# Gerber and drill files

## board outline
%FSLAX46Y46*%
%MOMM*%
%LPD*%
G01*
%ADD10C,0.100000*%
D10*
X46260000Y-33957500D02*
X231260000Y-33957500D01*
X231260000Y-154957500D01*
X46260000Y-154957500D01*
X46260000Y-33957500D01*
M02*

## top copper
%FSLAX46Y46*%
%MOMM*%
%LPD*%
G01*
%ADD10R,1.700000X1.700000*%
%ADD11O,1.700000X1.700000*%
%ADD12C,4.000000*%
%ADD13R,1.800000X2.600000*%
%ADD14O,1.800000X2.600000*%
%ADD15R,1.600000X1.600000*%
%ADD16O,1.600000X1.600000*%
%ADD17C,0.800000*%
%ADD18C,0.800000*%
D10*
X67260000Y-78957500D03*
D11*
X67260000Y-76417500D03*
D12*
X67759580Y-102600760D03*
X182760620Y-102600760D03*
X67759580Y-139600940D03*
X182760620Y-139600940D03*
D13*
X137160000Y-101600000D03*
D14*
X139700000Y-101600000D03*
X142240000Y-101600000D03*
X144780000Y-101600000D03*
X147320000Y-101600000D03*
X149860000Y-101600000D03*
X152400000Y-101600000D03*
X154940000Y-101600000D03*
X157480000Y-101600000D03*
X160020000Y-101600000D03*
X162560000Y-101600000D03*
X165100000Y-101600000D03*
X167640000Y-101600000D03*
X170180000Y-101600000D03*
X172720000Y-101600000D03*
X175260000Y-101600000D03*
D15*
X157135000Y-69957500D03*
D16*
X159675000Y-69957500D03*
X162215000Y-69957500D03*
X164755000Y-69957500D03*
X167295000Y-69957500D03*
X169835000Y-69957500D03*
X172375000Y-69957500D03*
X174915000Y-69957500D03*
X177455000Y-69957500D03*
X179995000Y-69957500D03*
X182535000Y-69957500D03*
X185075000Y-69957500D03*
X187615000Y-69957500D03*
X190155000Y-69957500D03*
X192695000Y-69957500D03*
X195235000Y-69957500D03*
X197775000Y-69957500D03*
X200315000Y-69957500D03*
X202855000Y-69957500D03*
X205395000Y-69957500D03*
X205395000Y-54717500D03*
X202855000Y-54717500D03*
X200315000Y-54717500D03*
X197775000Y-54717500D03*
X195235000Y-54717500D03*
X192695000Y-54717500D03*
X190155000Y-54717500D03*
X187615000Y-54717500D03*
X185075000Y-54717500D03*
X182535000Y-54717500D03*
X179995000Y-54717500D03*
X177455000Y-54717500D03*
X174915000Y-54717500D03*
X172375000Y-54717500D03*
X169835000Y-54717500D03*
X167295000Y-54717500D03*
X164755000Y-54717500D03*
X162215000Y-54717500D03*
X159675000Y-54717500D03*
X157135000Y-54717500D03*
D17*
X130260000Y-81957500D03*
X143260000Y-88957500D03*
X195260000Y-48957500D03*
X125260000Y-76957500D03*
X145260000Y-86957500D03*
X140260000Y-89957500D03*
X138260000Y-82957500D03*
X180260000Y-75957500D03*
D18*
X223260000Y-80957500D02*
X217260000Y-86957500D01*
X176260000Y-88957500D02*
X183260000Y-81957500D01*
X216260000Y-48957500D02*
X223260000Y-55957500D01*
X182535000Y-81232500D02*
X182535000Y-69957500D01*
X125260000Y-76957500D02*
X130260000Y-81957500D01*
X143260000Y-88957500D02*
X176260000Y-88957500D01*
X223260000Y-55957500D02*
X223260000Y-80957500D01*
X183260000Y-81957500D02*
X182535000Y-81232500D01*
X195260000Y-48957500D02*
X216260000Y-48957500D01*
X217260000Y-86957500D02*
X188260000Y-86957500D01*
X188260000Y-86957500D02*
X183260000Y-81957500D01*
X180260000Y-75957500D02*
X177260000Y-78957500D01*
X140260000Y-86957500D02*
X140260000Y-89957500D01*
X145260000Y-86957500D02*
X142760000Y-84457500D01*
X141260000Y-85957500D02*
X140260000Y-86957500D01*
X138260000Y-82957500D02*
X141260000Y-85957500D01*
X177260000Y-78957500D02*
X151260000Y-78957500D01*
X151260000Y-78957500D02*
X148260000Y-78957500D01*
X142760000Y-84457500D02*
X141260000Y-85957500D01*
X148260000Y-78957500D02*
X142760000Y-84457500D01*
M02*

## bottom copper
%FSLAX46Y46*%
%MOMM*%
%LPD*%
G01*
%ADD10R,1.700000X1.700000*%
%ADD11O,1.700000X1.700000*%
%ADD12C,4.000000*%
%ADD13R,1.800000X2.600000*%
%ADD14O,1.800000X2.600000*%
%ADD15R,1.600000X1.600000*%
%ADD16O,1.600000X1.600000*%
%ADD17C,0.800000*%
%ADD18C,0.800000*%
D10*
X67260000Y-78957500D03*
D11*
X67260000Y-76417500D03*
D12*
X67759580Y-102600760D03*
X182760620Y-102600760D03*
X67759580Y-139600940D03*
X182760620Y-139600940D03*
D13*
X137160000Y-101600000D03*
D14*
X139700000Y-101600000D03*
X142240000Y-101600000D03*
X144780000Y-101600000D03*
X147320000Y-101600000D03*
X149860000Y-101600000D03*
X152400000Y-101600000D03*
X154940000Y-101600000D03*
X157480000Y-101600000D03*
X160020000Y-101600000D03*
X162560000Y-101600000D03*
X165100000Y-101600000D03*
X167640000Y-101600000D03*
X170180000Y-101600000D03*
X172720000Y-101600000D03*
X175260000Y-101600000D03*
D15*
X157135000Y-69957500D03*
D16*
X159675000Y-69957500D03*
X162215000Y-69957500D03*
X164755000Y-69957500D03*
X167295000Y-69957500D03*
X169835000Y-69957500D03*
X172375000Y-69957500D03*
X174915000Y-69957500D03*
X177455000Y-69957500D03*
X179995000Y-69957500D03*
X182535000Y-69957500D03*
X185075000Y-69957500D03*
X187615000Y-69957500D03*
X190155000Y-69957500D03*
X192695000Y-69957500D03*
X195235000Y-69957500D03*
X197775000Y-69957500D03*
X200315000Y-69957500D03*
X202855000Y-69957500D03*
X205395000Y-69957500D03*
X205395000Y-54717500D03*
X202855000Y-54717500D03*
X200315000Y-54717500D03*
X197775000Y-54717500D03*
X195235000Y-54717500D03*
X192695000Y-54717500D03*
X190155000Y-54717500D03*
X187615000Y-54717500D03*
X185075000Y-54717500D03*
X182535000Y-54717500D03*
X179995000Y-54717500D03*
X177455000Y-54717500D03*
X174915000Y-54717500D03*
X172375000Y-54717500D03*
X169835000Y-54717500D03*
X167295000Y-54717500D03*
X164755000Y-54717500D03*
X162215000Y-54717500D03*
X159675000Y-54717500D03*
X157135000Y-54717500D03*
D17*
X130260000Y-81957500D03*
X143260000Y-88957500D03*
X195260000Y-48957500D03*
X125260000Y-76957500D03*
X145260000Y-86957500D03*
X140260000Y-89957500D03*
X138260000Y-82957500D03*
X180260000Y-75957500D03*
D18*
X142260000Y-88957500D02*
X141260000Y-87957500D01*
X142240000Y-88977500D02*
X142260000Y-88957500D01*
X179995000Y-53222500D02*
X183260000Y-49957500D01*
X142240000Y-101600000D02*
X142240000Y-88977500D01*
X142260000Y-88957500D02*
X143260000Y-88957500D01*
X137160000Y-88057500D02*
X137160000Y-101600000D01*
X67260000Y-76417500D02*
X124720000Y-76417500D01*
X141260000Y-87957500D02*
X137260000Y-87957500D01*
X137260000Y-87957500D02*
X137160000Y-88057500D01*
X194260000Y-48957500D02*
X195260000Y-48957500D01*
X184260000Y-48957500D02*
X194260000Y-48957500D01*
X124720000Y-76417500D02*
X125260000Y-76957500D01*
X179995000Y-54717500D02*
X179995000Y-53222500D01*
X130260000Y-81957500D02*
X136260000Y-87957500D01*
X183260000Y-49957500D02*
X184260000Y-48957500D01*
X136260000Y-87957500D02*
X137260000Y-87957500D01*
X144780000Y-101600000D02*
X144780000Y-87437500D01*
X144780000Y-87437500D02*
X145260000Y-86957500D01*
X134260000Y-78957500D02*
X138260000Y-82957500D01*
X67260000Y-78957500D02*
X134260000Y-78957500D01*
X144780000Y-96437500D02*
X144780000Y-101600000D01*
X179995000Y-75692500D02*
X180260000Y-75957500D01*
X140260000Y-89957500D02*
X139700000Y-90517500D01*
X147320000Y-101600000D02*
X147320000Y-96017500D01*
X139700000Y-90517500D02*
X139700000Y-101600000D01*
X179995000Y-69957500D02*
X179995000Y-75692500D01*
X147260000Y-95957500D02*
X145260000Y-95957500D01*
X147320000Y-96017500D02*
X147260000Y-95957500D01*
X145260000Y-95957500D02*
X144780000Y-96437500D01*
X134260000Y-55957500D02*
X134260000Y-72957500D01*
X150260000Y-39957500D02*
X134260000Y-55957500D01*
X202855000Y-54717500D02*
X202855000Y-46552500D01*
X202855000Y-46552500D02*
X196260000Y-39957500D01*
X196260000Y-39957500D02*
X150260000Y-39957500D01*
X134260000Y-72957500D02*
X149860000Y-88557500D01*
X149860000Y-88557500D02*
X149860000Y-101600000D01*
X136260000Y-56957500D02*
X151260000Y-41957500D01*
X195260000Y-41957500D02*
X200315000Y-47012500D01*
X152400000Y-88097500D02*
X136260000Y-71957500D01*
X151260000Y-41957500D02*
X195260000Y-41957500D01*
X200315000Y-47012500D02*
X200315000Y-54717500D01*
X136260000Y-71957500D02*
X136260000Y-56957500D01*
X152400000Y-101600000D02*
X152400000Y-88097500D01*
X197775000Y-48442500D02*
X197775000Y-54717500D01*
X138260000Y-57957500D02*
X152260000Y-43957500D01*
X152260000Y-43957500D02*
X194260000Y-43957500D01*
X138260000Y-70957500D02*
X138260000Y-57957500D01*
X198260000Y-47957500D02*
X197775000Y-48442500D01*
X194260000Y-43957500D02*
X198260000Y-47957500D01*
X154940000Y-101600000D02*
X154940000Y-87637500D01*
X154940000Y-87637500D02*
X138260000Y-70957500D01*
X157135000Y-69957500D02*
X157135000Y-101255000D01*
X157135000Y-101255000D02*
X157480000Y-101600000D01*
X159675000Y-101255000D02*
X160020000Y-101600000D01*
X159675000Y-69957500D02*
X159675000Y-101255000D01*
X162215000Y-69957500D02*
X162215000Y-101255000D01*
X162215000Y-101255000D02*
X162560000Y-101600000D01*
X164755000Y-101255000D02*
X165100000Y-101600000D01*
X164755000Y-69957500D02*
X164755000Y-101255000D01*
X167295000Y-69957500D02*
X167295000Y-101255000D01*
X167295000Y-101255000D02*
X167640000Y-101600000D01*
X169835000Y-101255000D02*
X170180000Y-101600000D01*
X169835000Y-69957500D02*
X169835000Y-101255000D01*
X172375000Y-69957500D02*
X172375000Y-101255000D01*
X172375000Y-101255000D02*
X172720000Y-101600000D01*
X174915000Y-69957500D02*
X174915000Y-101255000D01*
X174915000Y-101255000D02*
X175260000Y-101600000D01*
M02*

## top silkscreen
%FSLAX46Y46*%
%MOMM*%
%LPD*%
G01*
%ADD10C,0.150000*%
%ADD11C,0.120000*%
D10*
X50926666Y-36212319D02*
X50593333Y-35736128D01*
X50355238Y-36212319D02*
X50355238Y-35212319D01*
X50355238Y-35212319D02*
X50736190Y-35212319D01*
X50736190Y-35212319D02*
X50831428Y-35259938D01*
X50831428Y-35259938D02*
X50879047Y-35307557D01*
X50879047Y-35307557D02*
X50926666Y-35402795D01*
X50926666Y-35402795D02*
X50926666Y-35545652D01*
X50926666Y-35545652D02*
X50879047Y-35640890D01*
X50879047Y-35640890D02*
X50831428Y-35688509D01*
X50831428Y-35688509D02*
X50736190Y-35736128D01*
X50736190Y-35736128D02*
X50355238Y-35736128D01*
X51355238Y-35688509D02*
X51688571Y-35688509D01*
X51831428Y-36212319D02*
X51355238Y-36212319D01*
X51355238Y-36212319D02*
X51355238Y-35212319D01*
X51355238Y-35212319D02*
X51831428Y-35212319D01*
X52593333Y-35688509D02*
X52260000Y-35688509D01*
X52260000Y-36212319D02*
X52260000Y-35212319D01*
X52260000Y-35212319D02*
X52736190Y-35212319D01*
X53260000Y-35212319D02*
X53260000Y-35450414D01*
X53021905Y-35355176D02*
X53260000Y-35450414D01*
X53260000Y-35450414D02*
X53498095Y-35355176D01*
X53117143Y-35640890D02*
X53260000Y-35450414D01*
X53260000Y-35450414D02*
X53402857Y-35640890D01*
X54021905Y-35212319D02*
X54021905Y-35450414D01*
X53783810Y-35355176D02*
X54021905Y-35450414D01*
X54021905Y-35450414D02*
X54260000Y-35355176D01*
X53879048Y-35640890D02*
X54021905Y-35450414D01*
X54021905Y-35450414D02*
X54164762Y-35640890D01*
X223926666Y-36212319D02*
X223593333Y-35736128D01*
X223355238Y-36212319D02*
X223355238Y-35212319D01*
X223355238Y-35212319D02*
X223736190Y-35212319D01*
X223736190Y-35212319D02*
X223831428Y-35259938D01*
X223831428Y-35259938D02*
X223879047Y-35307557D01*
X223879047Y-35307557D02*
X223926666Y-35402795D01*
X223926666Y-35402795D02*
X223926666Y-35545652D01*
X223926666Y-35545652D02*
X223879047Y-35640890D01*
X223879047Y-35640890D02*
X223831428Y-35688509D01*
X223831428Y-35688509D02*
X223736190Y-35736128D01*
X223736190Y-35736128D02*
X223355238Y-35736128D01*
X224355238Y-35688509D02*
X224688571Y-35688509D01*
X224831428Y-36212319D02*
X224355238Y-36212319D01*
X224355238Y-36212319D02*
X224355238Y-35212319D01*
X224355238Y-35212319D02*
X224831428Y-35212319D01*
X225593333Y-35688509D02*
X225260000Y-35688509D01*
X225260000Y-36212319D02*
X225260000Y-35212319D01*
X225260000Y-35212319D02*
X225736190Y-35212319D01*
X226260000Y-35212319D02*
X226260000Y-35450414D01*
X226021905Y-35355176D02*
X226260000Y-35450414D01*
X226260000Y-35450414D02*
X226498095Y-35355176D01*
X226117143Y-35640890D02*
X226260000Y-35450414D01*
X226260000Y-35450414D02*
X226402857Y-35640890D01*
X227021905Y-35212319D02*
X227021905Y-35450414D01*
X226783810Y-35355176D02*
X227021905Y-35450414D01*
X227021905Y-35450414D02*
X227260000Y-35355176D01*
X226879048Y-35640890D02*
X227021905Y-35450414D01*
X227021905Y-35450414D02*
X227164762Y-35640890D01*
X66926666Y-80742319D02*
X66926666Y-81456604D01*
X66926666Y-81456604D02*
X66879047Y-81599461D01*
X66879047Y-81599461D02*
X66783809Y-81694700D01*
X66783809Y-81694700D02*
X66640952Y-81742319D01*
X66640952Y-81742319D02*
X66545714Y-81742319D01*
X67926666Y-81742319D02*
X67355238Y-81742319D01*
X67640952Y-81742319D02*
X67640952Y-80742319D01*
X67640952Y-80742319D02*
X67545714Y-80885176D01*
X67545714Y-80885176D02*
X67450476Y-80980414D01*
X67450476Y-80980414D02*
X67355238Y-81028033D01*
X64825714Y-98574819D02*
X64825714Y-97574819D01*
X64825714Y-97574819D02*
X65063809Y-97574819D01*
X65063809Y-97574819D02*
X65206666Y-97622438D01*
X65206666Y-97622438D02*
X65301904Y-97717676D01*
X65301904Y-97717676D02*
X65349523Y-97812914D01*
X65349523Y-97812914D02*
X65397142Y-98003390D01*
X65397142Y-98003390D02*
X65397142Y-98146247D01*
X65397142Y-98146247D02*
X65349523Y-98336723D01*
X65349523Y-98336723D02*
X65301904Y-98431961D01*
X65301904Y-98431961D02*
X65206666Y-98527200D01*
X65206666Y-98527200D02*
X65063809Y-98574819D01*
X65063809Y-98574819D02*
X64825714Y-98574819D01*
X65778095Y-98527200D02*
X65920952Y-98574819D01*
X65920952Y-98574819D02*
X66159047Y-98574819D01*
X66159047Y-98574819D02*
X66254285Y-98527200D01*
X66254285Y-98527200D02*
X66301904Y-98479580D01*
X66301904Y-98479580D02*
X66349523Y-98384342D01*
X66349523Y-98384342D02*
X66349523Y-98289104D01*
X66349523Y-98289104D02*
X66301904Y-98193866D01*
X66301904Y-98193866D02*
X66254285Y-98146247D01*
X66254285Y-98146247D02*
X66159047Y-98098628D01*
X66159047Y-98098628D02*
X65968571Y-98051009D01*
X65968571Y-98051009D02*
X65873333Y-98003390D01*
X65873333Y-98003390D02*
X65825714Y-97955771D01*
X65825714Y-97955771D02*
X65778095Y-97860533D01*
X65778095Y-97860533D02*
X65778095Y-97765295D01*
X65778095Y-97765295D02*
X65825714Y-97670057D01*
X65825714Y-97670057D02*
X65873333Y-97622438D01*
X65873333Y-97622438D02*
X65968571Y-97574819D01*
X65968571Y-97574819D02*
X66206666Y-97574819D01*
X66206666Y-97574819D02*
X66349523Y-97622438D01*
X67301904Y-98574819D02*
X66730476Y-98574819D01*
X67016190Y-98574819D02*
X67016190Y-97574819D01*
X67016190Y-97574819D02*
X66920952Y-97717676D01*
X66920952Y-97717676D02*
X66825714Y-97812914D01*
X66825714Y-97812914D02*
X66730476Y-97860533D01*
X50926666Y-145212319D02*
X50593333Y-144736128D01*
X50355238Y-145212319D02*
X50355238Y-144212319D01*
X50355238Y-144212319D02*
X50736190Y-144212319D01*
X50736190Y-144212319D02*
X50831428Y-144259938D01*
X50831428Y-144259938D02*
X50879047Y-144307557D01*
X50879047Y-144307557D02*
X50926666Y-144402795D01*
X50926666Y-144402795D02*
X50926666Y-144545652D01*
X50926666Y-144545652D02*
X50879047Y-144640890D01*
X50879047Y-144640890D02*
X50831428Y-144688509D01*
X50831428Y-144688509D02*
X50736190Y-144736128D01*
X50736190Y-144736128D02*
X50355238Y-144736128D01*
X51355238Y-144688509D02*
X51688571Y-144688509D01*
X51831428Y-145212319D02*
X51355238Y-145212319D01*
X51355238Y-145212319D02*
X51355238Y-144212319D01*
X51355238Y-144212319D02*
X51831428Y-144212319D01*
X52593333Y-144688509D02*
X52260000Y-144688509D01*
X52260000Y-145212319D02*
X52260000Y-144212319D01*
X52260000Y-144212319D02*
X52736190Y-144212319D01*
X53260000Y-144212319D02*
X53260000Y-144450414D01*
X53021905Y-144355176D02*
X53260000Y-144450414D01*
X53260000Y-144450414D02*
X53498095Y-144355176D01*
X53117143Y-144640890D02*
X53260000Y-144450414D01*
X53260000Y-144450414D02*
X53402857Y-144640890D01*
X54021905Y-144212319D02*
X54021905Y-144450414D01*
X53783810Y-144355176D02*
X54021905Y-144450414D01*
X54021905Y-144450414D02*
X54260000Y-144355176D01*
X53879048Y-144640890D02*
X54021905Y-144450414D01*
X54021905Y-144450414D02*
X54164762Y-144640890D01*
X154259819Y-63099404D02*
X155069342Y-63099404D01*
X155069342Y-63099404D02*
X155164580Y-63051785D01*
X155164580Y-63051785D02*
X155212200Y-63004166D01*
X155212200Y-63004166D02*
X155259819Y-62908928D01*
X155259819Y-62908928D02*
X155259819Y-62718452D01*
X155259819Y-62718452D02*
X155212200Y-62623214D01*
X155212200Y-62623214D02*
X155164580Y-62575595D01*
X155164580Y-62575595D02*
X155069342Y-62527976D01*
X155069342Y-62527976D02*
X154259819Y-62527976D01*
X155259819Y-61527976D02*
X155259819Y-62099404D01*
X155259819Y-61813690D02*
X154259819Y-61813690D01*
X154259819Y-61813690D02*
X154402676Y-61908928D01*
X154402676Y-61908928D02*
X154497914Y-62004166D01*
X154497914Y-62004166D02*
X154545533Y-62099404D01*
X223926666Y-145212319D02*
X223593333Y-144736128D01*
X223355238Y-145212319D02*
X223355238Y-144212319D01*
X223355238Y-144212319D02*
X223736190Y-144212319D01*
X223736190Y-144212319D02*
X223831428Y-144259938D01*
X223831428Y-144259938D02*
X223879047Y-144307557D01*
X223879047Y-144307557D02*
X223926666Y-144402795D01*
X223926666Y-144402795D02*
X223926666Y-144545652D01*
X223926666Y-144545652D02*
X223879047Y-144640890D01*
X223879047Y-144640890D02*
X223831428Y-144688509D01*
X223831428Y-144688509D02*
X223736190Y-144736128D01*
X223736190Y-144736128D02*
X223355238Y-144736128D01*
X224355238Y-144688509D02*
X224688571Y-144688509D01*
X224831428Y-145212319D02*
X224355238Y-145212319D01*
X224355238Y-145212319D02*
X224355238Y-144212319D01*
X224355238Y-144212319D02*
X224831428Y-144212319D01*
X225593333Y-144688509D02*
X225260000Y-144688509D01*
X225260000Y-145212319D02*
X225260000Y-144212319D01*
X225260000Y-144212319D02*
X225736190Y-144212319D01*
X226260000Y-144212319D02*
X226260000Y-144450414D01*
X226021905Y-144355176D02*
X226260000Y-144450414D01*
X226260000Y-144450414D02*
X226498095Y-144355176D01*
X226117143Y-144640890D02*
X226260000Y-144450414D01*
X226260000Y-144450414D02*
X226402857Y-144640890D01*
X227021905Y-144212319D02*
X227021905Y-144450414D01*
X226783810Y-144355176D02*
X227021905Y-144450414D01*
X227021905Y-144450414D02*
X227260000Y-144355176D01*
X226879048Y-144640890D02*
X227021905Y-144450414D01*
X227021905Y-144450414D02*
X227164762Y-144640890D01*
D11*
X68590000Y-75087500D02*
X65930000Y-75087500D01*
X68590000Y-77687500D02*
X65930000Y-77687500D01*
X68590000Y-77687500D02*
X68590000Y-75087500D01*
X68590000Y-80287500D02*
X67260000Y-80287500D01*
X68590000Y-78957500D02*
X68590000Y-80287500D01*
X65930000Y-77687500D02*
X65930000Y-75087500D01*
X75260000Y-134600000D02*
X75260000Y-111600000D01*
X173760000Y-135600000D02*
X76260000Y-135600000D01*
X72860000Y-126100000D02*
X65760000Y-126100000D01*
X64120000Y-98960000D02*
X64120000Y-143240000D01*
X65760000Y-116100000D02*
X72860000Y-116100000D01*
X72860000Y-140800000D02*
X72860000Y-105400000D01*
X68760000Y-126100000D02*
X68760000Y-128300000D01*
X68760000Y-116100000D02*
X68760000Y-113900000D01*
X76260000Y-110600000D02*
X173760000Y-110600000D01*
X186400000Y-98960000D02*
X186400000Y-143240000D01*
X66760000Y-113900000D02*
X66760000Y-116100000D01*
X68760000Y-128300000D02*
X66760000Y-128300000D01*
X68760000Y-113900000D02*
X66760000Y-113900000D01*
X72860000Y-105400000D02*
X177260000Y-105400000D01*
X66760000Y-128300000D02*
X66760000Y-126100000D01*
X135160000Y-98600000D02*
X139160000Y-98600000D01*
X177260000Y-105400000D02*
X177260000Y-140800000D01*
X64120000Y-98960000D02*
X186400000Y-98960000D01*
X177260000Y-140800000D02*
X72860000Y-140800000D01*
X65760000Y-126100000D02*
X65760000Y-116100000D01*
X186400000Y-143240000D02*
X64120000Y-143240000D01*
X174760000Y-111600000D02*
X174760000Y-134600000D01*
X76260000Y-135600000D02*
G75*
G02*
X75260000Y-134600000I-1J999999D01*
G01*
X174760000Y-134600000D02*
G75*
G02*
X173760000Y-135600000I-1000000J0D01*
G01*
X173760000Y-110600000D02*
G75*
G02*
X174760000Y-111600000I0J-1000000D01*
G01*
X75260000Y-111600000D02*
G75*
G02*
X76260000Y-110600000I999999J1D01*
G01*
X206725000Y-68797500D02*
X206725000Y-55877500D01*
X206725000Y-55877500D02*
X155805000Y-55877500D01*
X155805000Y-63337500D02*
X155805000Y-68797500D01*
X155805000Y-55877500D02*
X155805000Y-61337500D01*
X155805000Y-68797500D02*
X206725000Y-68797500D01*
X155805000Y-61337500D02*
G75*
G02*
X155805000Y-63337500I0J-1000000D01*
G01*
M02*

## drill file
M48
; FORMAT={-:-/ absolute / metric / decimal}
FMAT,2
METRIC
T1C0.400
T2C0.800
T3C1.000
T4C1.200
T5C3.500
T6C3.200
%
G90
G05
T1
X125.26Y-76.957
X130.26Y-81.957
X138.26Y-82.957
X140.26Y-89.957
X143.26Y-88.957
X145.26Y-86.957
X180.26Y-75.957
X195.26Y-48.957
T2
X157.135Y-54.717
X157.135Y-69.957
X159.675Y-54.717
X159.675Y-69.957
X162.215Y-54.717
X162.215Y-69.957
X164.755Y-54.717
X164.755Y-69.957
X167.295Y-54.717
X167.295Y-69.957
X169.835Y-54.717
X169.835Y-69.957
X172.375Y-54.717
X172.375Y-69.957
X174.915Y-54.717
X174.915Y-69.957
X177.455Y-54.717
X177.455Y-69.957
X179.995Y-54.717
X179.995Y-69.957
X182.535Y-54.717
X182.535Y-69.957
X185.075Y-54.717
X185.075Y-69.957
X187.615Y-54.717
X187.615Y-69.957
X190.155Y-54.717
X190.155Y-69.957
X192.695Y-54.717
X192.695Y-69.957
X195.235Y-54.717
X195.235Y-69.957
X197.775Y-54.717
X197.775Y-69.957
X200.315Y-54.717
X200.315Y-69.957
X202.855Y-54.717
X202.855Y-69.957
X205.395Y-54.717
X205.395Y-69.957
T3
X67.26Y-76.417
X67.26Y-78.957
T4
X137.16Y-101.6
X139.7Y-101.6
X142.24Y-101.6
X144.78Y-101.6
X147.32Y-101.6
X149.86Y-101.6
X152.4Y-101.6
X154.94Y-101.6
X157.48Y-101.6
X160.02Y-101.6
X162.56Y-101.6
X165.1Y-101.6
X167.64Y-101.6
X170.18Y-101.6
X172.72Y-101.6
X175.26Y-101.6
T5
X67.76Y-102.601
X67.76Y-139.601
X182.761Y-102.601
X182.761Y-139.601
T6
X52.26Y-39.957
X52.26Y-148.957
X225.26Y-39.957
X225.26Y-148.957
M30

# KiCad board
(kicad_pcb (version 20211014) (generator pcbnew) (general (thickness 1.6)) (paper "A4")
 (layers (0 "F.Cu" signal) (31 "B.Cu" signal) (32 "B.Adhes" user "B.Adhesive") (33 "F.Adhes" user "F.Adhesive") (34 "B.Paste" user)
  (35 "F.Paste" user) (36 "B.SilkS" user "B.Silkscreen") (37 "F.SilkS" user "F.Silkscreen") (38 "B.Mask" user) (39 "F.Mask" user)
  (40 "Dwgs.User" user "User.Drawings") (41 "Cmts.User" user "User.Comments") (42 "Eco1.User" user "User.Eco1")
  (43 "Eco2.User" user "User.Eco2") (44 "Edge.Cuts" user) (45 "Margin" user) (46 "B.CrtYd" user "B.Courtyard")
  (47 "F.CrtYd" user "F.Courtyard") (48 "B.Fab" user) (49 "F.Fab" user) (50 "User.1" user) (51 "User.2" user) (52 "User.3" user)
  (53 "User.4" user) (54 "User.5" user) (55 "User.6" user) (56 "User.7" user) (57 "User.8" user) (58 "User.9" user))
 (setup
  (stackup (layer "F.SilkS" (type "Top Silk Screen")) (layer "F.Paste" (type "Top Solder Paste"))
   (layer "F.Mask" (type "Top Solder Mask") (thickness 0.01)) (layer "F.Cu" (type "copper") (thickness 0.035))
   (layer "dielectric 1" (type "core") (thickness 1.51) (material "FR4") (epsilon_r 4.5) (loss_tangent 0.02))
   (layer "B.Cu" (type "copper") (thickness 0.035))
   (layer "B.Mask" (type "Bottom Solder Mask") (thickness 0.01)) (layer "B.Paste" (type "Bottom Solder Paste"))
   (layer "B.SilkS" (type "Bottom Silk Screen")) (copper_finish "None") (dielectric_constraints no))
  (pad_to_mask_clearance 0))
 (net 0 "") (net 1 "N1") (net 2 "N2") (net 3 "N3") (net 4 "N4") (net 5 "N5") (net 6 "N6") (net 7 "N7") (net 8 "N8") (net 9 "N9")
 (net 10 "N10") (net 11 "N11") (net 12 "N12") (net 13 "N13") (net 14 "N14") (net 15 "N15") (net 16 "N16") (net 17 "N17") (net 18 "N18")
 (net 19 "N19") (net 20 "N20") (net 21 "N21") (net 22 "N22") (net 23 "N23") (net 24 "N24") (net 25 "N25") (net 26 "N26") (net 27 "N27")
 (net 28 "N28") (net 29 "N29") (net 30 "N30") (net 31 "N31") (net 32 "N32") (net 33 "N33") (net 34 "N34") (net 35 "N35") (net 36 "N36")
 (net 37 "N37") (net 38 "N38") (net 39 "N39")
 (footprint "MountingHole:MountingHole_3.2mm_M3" (layer "F.Cu") (at 52.26 39.9575)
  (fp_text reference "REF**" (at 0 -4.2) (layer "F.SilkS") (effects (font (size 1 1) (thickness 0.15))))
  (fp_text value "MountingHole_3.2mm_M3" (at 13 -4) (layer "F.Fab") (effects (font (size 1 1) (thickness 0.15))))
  (pad "" np_thru_hole circle (at 0 0) (size 3.2 3.2) (drill 3.2) (layers *.Cu *.Mask)))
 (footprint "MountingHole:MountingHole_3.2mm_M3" (layer "F.Cu") (at 225.26 39.9575)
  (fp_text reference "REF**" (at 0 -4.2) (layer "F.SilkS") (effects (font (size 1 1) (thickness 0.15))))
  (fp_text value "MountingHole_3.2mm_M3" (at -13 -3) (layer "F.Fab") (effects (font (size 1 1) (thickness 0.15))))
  (pad "" np_thru_hole circle (at 0 0) (size 3.2 3.2) (drill 3.2) (layers *.Cu *.Mask)))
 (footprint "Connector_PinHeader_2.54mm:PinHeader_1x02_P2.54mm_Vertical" (layer "F.Cu") (at 67.26 78.9575 180)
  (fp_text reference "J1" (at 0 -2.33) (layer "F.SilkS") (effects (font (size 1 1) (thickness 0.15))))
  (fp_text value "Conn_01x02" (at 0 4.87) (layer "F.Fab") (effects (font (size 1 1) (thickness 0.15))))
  (fp_line (start -1.33 3.87) (end 1.33 3.87) (layer "F.SilkS") (width 0.12))
  (fp_line (start -1.33 1.27) (end 1.33 1.27) (layer "F.SilkS") (width 0.12))
  (fp_line (start -1.33 1.27) (end -1.33 3.87) (layer "F.SilkS") (width 0.12))
  (fp_line (start -1.33 -1.33) (end 0 -1.33) (layer "F.SilkS") (width 0.12))
  (fp_line (start -1.33 0) (end -1.33 -1.33) (layer "F.SilkS") (width 0.12))
  (fp_line (start 1.33 1.27) (end 1.33 3.87) (layer "F.SilkS") (width 0.12))
  (pad "1" thru_hole rect (at 0 0 180) (size 1.7 1.7) (drill 1) (layers *.Cu *.Mask) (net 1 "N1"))
  (pad "2" thru_hole oval (at 0 2.54 180) (size 1.7 1.7) (drill 1) (layers *.Cu *.Mask) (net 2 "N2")))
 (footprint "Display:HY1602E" (layer "F.Cu") (at 137.16 101.6)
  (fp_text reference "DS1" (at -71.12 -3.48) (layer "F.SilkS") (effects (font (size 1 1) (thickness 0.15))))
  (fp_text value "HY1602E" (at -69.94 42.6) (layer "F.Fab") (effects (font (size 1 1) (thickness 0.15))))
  (fp_line (start -61.9 33) (end -61.9 10) (layer "F.SilkS") (width 0.12))
  (fp_line (start 36.6 34) (end -60.9 34) (layer "F.SilkS") (width 0.12))
  (fp_line (start -64.3 24.5) (end -71.4 24.5) (layer "F.SilkS") (width 0.12))
  (fp_line (start -73.04 -2.64) (end -73.04 41.64) (layer "F.SilkS") (width 0.12))
  (fp_line (start -71.4 14.5) (end -64.3 14.5) (layer "F.SilkS") (width 0.12))
  (fp_line (start -64.3 39.2) (end -64.3 3.8) (layer "F.SilkS") (width 0.12))
  (fp_line (start -68.4 24.5) (end -68.4 26.7) (layer "F.SilkS") (width 0.12))
  (fp_line (start -68.4 14.5) (end -68.4 12.3) (layer "F.SilkS") (width 0.12))
  (fp_line (start -60.9 9) (end 36.6 9) (layer "F.SilkS") (width 0.12))
  (fp_line (start 49.24 -2.64) (end 49.24 41.64) (layer "F.SilkS") (width 0.12))
  (fp_line (start -70.4 12.3) (end -70.4 14.5) (layer "F.SilkS") (width 0.12))
  (fp_line (start -68.4 26.7) (end -70.4 26.7) (layer "F.SilkS") (width 0.12))
  (fp_line (start -68.4 12.3) (end -70.4 12.3) (layer "F.SilkS") (width 0.12))
  (fp_line (start -64.3 3.8) (end 40.1 3.8) (layer "F.SilkS") (width 0.12))
  (fp_line (start -70.4 26.7) (end -70.4 24.5) (layer "F.SilkS") (width 0.12))
  (fp_line (start -2 -3) (end 2 -3) (layer "F.SilkS") (width 0.12))
  (fp_line (start 40.1 3.8) (end 40.1 39.2) (layer "F.SilkS") (width 0.12))
  (fp_line (start -73.04 -2.64) (end 49.24 -2.64) (layer "F.SilkS") (width 0.12))
  (fp_line (start 40.1 39.2) (end -64.3 39.2) (layer "F.SilkS") (width 0.12))
  (fp_line (start -71.4 24.5) (end -71.4 14.5) (layer "F.SilkS") (width 0.12))
  (fp_line (start 49.24 41.64) (end -73.04 41.64) (layer "F.SilkS") (width 0.12))
  (fp_line (start 37.6 10) (end 37.6 33) (layer "F.SilkS") (width 0.12))
  (fp_arc (start -60.9 34) (mid -61.607107 33.707107) (end -61.9 33) (layer "F.SilkS") (width 0.12))
  (fp_arc (start 37.6 33) (mid 37.307107 33.707107) (end 36.6 34) (layer "F.SilkS") (width 0.12))
  (fp_arc (start 36.6 9) (mid 37.307107 9.292893) (end 37.6 10) (layer "F.SilkS") (width 0.12))
  (fp_arc (start -61.9 10) (mid -61.607107 9.292893) (end -60.9 9) (layer "F.SilkS") (width 0.12))
  (pad "" thru_hole circle (at -69.40042 1.00076 180) (size 4 4) (drill 3.5) (layers *.Cu *.Mask))
  (pad "" thru_hole circle (at 45.60062 1.00076 180) (size 4 4) (drill 3.5) (layers *.Cu *.Mask))
  (pad "" thru_hole circle (at -69.40042 38.00094 180) (size 4 4) (drill 3.5) (layers *.Cu *.Mask))
  (pad "" thru_hole circle (at 45.60062 38.00094 180) (size 4 4) (drill 3.5) (layers *.Cu *.Mask))
  (pad "1" thru_hole rect (at 0 0 180) (size 1.8 2.6) (drill 1.2) (layers *.Cu *.Mask) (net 2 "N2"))
  (pad "2" thru_hole oval (at 2.54 0 180) (size 1.8 2.6) (drill 1.2) (layers *.Cu *.Mask) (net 1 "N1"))
  (pad "3" thru_hole oval (at 5.08 0 180) (size 1.8 2.6) (drill 1.2) (layers *.Cu *.Mask) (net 2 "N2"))
  (pad "4" thru_hole oval (at 7.62 0 180) (size 1.8 2.6) (drill 1.2) (layers *.Cu *.Mask) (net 1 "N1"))
  (pad "5" thru_hole oval (at 10.16 0 180) (size 1.8 2.6) (drill 1.2) (layers *.Cu *.Mask) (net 1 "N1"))
  (pad "6" thru_hole oval (at 12.7 0 180) (size 1.8 2.6) (drill 1.2) (layers *.Cu *.Mask) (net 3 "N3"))
  (pad "7" thru_hole oval (at 15.24 0 180) (size 1.8 2.6) (drill 1.2) (layers *.Cu *.Mask) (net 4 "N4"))
  (pad "8" thru_hole oval (at 17.78 0 180) (size 1.8 2.6) (drill 1.2) (layers *.Cu *.Mask) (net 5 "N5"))
  (pad "9" thru_hole oval (at 20.32 0 180) (size 1.8 2.6) (drill 1.2) (layers *.Cu *.Mask) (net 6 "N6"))
  (pad "10" thru_hole oval (at 22.86 0 180) (size 1.8 2.6) (drill 1.2) (layers *.Cu *.Mask) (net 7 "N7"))
  (pad "11" thru_hole oval (at 25.4 0 180) (size 1.8 2.6) (drill 1.2) (layers *.Cu *.Mask) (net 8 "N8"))
  (pad "12" thru_hole oval (at 27.94 0 180) (size 1.8 2.6) (drill 1.2) (layers *.Cu *.Mask) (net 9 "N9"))
  (pad "13" thru_hole oval (at 30.48 0 180) (size 1.8 2.6) (drill 1.2) (layers *.Cu *.Mask) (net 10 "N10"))
  (pad "14" thru_hole oval (at 33.02 0 180) (size 1.8 2.6) (drill 1.2) (layers *.Cu *.Mask) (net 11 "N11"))
  (pad "15" thru_hole oval (at 35.56 0 180) (size 1.8 2.6) (drill 1.2) (layers *.Cu *.Mask) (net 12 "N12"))
  (pad "16" thru_hole oval (at 38.1 0 180) (size 1.8 2.6) (drill 1.2) (layers *.Cu *.Mask) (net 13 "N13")))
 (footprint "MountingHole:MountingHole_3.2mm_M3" (layer "F.Cu") (at 52.26 148.9575)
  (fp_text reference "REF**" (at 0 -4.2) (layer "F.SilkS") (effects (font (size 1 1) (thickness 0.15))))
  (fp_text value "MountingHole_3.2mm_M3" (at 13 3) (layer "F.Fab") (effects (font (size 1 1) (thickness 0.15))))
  (pad "" np_thru_hole circle (at 0 0) (size 3.2 3.2) (drill 3.2) (layers *.Cu *.Mask)))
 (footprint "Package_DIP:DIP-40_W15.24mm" (layer "F.Cu") (at 157.135 69.9575 90)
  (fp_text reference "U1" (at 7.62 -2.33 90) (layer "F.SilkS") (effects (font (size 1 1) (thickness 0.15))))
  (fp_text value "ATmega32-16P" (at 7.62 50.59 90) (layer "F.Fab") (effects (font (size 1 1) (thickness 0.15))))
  (fp_line (start 1.16 49.59) (end 14.08 49.59) (layer "F.SilkS") (width 0.12))
  (fp_line (start 14.08 49.59) (end 14.08 -1.33) (layer "F.SilkS") (width 0.12))
  (fp_line (start 6.62 -1.33) (end 1.16 -1.33) (layer "F.SilkS") (width 0.12))
  (fp_line (start 14.08 -1.33) (end 8.62 -1.33) (layer "F.SilkS") (width 0.12))
  (fp_line (start 1.16 -1.33) (end 1.16 49.59) (layer "F.SilkS") (width 0.12))
  (fp_arc (start 8.62 -1.33) (mid 7.62 -0.33) (end 6.62 -1.33) (layer "F.SilkS") (width 0.12))
  (pad "1" thru_hole rect (at 0 0 90) (size 1.6 1.6) (drill 0.8) (layers *.Cu *.Mask) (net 6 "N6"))
  (pad "2" thru_hole oval (at 0 2.54 90) (size 1.6 1.6) (drill 0.8) (layers *.Cu *.Mask) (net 7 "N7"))
  (pad "3" thru_hole oval (at 0 5.08 90) (size 1.6 1.6) (drill 0.8) (layers *.Cu *.Mask) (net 8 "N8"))
  (pad "4" thru_hole oval (at 0 7.62 90) (size 1.6 1.6) (drill 0.8) (layers *.Cu *.Mask) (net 9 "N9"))
  (pad "5" thru_hole oval (at 0 10.16 90) (size 1.6 1.6) (drill 0.8) (layers *.Cu *.Mask) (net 10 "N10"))
  (pad "6" thru_hole oval (at 0 12.7 90) (size 1.6 1.6) (drill 0.8) (layers *.Cu *.Mask) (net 11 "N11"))
  (pad "7" thru_hole oval (at 0 15.24 90) (size 1.6 1.6) (drill 0.8) (layers *.Cu *.Mask) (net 12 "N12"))
  (pad "8" thru_hole oval (at 0 17.78 90) (size 1.6 1.6) (drill 0.8) (layers *.Cu *.Mask) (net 13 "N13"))
  (pad "9" thru_hole oval (at 0 20.32 90) (size 1.6 1.6) (drill 0.8) (layers *.Cu *.Mask) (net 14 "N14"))
  (pad "10" thru_hole oval (at 0 22.86 90) (size 1.6 1.6) (drill 0.8) (layers *.Cu *.Mask) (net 1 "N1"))
  (pad "11" thru_hole oval (at 0 25.4 90) (size 1.6 1.6) (drill 0.8) (layers *.Cu *.Mask) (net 2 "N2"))
  (pad "12" thru_hole oval (at 0 27.94 90) (size 1.6 1.6) (drill 0.8) (layers *.Cu *.Mask) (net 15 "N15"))
  (pad "13" thru_hole oval (at 0 30.48 90) (size 1.6 1.6) (drill 0.8) (layers *.Cu *.Mask) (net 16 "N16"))
  (pad "14" thru_hole oval (at 0 33.02 90) (size 1.6 1.6) (drill 0.8) (layers *.Cu *.Mask) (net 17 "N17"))
  (pad "15" thru_hole oval (at 0 35.56 90) (size 1.6 1.6) (drill 0.8) (layers *.Cu *.Mask) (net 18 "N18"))
  (pad "16" thru_hole oval (at 0 38.1 90) (size 1.6 1.6) (drill 0.8) (layers *.Cu *.Mask) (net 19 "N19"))
  (pad "17" thru_hole oval (at 0 40.64 90) (size 1.6 1.6) (drill 0.8) (layers *.Cu *.Mask) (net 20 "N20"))
  (pad "18" thru_hole oval (at 0 43.18 90) (size 1.6 1.6) (drill 0.8) (layers *.Cu *.Mask) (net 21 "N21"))
  (pad "19" thru_hole oval (at 0 45.72 90) (size 1.6 1.6) (drill 0.8) (layers *.Cu *.Mask) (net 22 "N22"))
  (pad "20" thru_hole oval (at 0 48.26 90) (size 1.6 1.6) (drill 0.8) (layers *.Cu *.Mask) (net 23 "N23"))
  (pad "21" thru_hole oval (at 15.24 48.26 90) (size 1.6 1.6) (drill 0.8) (layers *.Cu *.Mask) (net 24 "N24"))
  (pad "22" thru_hole oval (at 15.24 45.72 90) (size 1.6 1.6) (drill 0.8) (layers *.Cu *.Mask) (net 3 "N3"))
  (pad "23" thru_hole oval (at 15.24 43.18 90) (size 1.6 1.6) (drill 0.8) (layers *.Cu *.Mask) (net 4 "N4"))
  (pad "24" thru_hole oval (at 15.24 40.64 90) (size 1.6 1.6) (drill 0.8) (layers *.Cu *.Mask) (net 5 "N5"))
  (pad "25" thru_hole oval (at 15.24 38.1 90) (size 1.6 1.6) (drill 0.8) (layers *.Cu *.Mask) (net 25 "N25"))
  (pad "26" thru_hole oval (at 15.24 35.56 90) (size 1.6 1.6) (drill 0.8) (layers *.Cu *.Mask) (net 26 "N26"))
  (pad "27" thru_hole oval (at 15.24 33.02 90) (size 1.6 1.6) (drill 0.8) (layers *.Cu *.Mask) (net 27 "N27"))
  (pad "28" thru_hole oval (at 15.24 30.48 90) (size 1.6 1.6) (drill 0.8) (layers *.Cu *.Mask) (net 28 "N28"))
  (pad "29" thru_hole oval (at 15.24 27.94 90) (size 1.6 1.6) (drill 0.8) (layers *.Cu *.Mask) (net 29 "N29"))
  (pad "30" thru_hole oval (at 15.24 25.4 90) (size 1.6 1.6) (drill 0.8) (layers *.Cu *.Mask) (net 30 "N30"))
  (pad "31" thru_hole oval (at 15.24 22.86 90) (size 1.6 1.6) (drill 0.8) (layers *.Cu *.Mask) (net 2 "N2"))
  (pad "32" thru_hole oval (at 15.24 20.32 90) (size 1.6 1.6) (drill 0.8) (layers *.Cu *.Mask) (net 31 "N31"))
  (pad "33" thru_hole oval (at 15.24 17.78 90) (size 1.6 1.6) (drill 0.8) (layers *.Cu *.Mask) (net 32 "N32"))
  (pad "34" thru_hole oval (at 15.24 15.24 90) (size 1.6 1.6) (drill 0.8) (layers *.Cu *.Mask) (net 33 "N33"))
  (pad "35" thru_hole oval (at 15.24 12.7 90) (size 1.6 1.6) (drill 0.8) (layers *.Cu *.Mask) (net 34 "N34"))
  (pad "36" thru_hole oval (at 15.24 10.16 90) (size 1.6 1.6) (drill 0.8) (layers *.Cu *.Mask) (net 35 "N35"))
  (pad "37" thru_hole oval (at 15.24 7.62 90) (size 1.6 1.6) (drill 0.8) (layers *.Cu *.Mask) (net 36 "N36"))
  (pad "38" thru_hole oval (at 15.24 5.08 90) (size 1.6 1.6) (drill 0.8) (layers *.Cu *.Mask) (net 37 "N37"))
  (pad "39" thru_hole oval (at 15.24 2.54 90) (size 1.6 1.6) (drill 0.8) (layers *.Cu *.Mask) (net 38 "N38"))
  (pad "40" thru_hole oval (at 15.24 0 90) (size 1.6 1.6) (drill 0.8) (layers *.Cu *.Mask) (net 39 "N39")))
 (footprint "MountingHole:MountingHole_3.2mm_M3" (layer "F.Cu") (at 225.26 148.9575)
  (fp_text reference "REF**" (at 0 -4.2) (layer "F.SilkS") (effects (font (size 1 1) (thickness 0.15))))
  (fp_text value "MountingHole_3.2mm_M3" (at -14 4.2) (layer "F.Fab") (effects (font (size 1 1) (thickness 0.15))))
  (pad "" np_thru_hole circle (at 0 0) (size 3.2 3.2) (drill 3.2) (layers *.Cu *.Mask)))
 (gr_rect (start 231.26 33.9575) (end 46.26 154.9575) (layer "Edge.Cuts") (width 0.1) (fill none))
 (segment (start 223.26 80.9575) (end 217.26 86.9575) (width 0.8) (layer "F.Cu") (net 2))
 (segment (start 176.26 88.9575) (end 183.26 81.9575) (width 0.8) (layer "F.Cu") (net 2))
 (segment (start 216.26 48.9575) (end 223.26 55.9575) (width 0.8) (layer "F.Cu") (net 2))
 (segment (start 182.535 81.2325) (end 182.535 69.9575) (width 0.8) (layer "F.Cu") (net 2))
 (segment (start 125.26 76.9575) (end 130.26 81.9575) (width 0.8) (layer "F.Cu") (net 2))
 (segment (start 143.26 88.9575) (end 176.26 88.9575) (width 0.8) (layer "F.Cu") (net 2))
 (segment (start 223.26 55.9575) (end 223.26 80.9575) (width 0.8) (layer "F.Cu") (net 2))
 (segment (start 183.26 81.9575) (end 182.535 81.2325) (width 0.8) (layer "F.Cu") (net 2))
 (segment (start 195.26 48.9575) (end 216.26 48.9575) (width 0.8) (layer "F.Cu") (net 2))
 (segment (start 217.26 86.9575) (end 188.26 86.9575) (width 0.8) (layer "F.Cu") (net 2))
 (segment (start 188.26 86.9575) (end 183.26 81.9575) (width 0.8) (layer "F.Cu") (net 2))
 (via (at 130.26 81.9575) (size 0.8) (drill 0.4) (layers "F.Cu" "B.Cu") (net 2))
 (via (at 143.26 88.9575) (size 0.8) (drill 0.4) (layers "F.Cu" "B.Cu") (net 2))
 (via (at 195.26 48.9575) (size 0.8) (drill 0.4) (layers "F.Cu" "B.Cu") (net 2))
 (via (at 125.26 76.9575) (size 0.8) (drill 0.4) (layers "F.Cu" "B.Cu") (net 2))
 (segment (start 142.26 88.9575) (end 141.26 87.9575) (width 0.8) (layer "B.Cu") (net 2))
 (segment (start 142.24 88.9775) (end 142.26 88.9575) (width 0.8) (layer "B.Cu") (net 2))
 (segment (start 179.995 53.2225) (end 183.26 49.9575) (width 0.8) (layer "B.Cu") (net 2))
 (segment (start 142.24 101.6) (end 142.24 88.9775) (width 0.8) (layer "B.Cu") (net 2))
 (segment (start 142.26 88.9575) (end 143.26 88.9575) (width 0.8) (layer "B.Cu") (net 2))
 (segment (start 137.16 88.0575) (end 137.16 101.6) (width 0.8) (layer "B.Cu") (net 2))
 (segment (start 67.26 76.4175) (end 124.72 76.4175) (width 0.8) (layer "B.Cu") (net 2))
 (segment (start 141.26 87.9575) (end 137.26 87.9575) (width 0.8) (layer "B.Cu") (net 2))
 (segment (start 137.26 87.9575) (end 137.16 88.0575) (width 0.8) (layer "B.Cu") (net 2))
 (segment (start 194.26 48.9575) (end 195.26 48.9575) (width 0.8) (layer "B.Cu") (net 2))
 (segment (start 184.26 48.9575) (end 194.26 48.9575) (width 0.8) (layer "B.Cu") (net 2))
 (segment (start 124.72 76.4175) (end 125.26 76.9575) (width 0.8) (layer "B.Cu") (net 2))
 (segment (start 179.995 54.7175) (end 179.995 53.2225) (width 0.8) (layer "B.Cu") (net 2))
 (segment (start 130.26 81.9575) (end 136.26 87.9575) (width 0.8) (layer "B.Cu") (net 2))
 (segment (start 183.26 49.9575) (end 184.26 48.9575) (width 0.8) (layer "B.Cu") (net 2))
 (segment (start 136.26 87.9575) (end 137.26 87.9575) (width 0.8) (layer "B.Cu") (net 2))
 (segment (start 180.26 75.9575) (end 177.26 78.9575) (width 0.8) (layer "F.Cu") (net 1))
 (segment (start 140.26 86.9575) (end 140.26 89.9575) (width 0.8) (layer "F.Cu") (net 1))
 (segment (start 145.26 86.9575) (end 142.76 84.4575) (width 0.8) (layer "F.Cu") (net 1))
 (segment (start 141.26 85.9575) (end 140.26 86.9575) (width 0.8) (layer "F.Cu") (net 1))
 (segment (start 138.26 82.9575) (end 141.26 85.9575) (width 0.8) (layer "F.Cu") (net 1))
 (segment (start 177.26 78.9575) (end 151.26 78.9575) (width 0.8) (layer "F.Cu") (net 1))
 (segment (start 151.26 78.9575) (end 148.26 78.9575) (width 0.8) (layer "F.Cu") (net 1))
 (segment (start 142.76 84.4575) (end 141.26 85.9575) (width 0.8) (layer "F.Cu") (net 1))
 (segment (start 148.26 78.9575) (end 142.76 84.4575) (width 0.8) (layer "F.Cu") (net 1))
 (via (at 145.26 86.9575) (size 0.8) (drill 0.4) (layers "F.Cu" "B.Cu") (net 1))
 (via (at 140.26 89.9575) (size 0.8) (drill 0.4) (layers "F.Cu" "B.Cu") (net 1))
 (via (at 138.26 82.9575) (size 0.8) (drill 0.4) (layers "F.Cu" "B.Cu") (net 1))
 (via (at 180.26 75.9575) (size 0.8) (drill 0.4) (layers "F.Cu" "B.Cu") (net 1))
 (segment (start 144.78 101.6) (end 144.78 87.4375) (width 0.8) (layer "B.Cu") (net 1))
 (segment (start 144.78 87.4375) (end 145.26 86.9575) (width 0.8) (layer "B.Cu") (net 1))
 (segment (start 134.26 78.9575) (end 138.26 82.9575) (width 0.8) (layer "B.Cu") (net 1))
 (segment (start 67.26 78.9575) (end 134.26 78.9575) (width 0.8) (layer "B.Cu") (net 1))
 (segment (start 144.78 96.4375) (end 144.78 101.6) (width 0.8) (layer "B.Cu") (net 1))
 (segment (start 179.995 75.6925) (end 180.26 75.9575) (width 0.8) (layer "B.Cu") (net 1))
 (segment (start 140.26 89.9575) (end 139.7 90.5175) (width 0.8) (layer "B.Cu") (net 1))
 (segment (start 147.32 101.6) (end 147.32 96.0175) (width 0.8) (layer "B.Cu") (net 1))
 (segment (start 139.7 90.5175) (end 139.7 101.6) (width 0.8) (layer "B.Cu") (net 1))
 (segment (start 179.995 69.9575) (end 179.995 75.6925) (width 0.8) (layer "B.Cu") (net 1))
 (segment (start 147.26 95.9575) (end 145.26 95.9575) (width 0.8) (layer "B.Cu") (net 1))
 (segment (start 147.32 96.0175) (end 147.26 95.9575) (width 0.8) (layer "B.Cu") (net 1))
 (segment (start 145.26 95.9575) (end 144.78 96.4375) (width 0.8) (layer "B.Cu") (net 1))
 (segment (start 134.26 55.9575) (end 134.26 72.9575) (width 0.8) (layer "B.Cu") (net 3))
 (segment (start 150.26 39.9575) (end 134.26 55.9575) (width 0.8) (layer "B.Cu") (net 3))
 (segment (start 202.855 54.7175) (end 202.855 46.5525) (width 0.8) (layer "B.Cu") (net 3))
 (segment (start 202.855 46.5525) (end 196.26 39.9575) (width 0.8) (layer "B.Cu") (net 3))
 (segment (start 196.26 39.9575) (end 150.26 39.9575) (width 0.8) (layer "B.Cu") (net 3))
 (segment (start 134.26 72.9575) (end 149.86 88.5575) (width 0.8) (layer "B.Cu") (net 3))
 (segment (start 149.86 88.5575) (end 149.86 101.6) (width 0.8) (layer "B.Cu") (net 3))
 (segment (start 136.26 56.9575) (end 151.26 41.9575) (width 0.8) (layer "B.Cu") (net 4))
 (segment (start 195.26 41.9575) (end 200.315 47.0125) (width 0.8) (layer "B.Cu") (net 4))
 (segment (start 152.4 88.0975) (end 136.26 71.9575) (width 0.8) (layer "B.Cu") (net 4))
 (segment (start 151.26 41.9575) (end 195.26 41.9575) (width 0.8) (layer "B.Cu") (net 4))
 (segment (start 200.315 47.0125) (end 200.315 54.7175) (width 0.8) (layer "B.Cu") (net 4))
 (segment (start 136.26 71.9575) (end 136.26 56.9575) (width 0.8) (layer "B.Cu") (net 4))
 (segment (start 152.4 101.6) (end 152.4 88.0975) (width 0.8) (layer "B.Cu") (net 4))
 (segment (start 197.775 48.4425) (end 197.775 54.7175) (width 0.8) (layer "B.Cu") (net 5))
 (segment (start 138.26 57.9575) (end 152.26 43.9575) (width 0.8) (layer "B.Cu") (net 5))
 (segment (start 152.26 43.9575) (end 194.26 43.9575) (width 0.8) (layer "B.Cu") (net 5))
 (segment (start 138.26 70.9575) (end 138.26 57.9575) (width 0.8) (layer "B.Cu") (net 5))
 (segment (start 198.26 47.9575) (end 197.775 48.4425) (width 0.8) (layer "B.Cu") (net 5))
 (segment (start 194.26 43.9575) (end 198.26 47.9575) (width 0.8) (layer "B.Cu") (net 5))
 (segment (start 154.94 101.6) (end 154.94 87.6375) (width 0.8) (layer "B.Cu") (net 5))
 (segment (start 154.94 87.6375) (end 138.26 70.9575) (width 0.8) (layer "B.Cu") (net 5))
 (segment (start 157.135 69.9575) (end 157.135 101.255) (width 0.8) (layer "B.Cu") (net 6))
 (segment (start 157.135 101.255) (end 157.48 101.6) (width 0.8) (layer "B.Cu") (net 6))
 (segment (start 159.675 101.255) (end 160.02 101.6) (width 0.8) (layer "B.Cu") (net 7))
 (segment (start 159.675 69.9575) (end 159.675 101.255) (width 0.8) (layer "B.Cu") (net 7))
 (segment (start 162.215 69.9575) (end 162.215 101.255) (width 0.8) (layer "B.Cu") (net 8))
 (segment (start 162.215 101.255) (end 162.56 101.6) (width 0.8) (layer "B.Cu") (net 8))
 (segment (start 164.755 101.255) (end 165.1 101.6) (width 0.8) (layer "B.Cu") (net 9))
 (segment (start 164.755 69.9575) (end 164.755 101.255) (width 0.8) (layer "B.Cu") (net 9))
 (segment (start 167.295 69.9575) (end 167.295 101.255) (width 0.8) (layer "B.Cu") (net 10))
 (segment (start 167.295 101.255) (end 167.64 101.6) (width 0.8) (layer "B.Cu") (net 10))
 (segment (start 169.835 101.255) (end 170.18 101.6) (width 0.8) (layer "B.Cu") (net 11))
 (segment (start 169.835 69.9575) (end 169.835 101.255) (width 0.8) (layer "B.Cu") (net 11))
 (segment (start 172.375 69.9575) (end 172.375 101.255) (width 0.8) (layer "B.Cu") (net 12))
 (segment (start 172.375 101.255) (end 172.72 101.6) (width 0.8) (layer "B.Cu") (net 12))
 (segment (start 174.915 69.9575) (end 174.915 101.255) (width 0.8) (layer "B.Cu") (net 13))
 (segment (start 174.915 101.255) (end 175.26 101.6) (width 0.8) (layer "B.Cu") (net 13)))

